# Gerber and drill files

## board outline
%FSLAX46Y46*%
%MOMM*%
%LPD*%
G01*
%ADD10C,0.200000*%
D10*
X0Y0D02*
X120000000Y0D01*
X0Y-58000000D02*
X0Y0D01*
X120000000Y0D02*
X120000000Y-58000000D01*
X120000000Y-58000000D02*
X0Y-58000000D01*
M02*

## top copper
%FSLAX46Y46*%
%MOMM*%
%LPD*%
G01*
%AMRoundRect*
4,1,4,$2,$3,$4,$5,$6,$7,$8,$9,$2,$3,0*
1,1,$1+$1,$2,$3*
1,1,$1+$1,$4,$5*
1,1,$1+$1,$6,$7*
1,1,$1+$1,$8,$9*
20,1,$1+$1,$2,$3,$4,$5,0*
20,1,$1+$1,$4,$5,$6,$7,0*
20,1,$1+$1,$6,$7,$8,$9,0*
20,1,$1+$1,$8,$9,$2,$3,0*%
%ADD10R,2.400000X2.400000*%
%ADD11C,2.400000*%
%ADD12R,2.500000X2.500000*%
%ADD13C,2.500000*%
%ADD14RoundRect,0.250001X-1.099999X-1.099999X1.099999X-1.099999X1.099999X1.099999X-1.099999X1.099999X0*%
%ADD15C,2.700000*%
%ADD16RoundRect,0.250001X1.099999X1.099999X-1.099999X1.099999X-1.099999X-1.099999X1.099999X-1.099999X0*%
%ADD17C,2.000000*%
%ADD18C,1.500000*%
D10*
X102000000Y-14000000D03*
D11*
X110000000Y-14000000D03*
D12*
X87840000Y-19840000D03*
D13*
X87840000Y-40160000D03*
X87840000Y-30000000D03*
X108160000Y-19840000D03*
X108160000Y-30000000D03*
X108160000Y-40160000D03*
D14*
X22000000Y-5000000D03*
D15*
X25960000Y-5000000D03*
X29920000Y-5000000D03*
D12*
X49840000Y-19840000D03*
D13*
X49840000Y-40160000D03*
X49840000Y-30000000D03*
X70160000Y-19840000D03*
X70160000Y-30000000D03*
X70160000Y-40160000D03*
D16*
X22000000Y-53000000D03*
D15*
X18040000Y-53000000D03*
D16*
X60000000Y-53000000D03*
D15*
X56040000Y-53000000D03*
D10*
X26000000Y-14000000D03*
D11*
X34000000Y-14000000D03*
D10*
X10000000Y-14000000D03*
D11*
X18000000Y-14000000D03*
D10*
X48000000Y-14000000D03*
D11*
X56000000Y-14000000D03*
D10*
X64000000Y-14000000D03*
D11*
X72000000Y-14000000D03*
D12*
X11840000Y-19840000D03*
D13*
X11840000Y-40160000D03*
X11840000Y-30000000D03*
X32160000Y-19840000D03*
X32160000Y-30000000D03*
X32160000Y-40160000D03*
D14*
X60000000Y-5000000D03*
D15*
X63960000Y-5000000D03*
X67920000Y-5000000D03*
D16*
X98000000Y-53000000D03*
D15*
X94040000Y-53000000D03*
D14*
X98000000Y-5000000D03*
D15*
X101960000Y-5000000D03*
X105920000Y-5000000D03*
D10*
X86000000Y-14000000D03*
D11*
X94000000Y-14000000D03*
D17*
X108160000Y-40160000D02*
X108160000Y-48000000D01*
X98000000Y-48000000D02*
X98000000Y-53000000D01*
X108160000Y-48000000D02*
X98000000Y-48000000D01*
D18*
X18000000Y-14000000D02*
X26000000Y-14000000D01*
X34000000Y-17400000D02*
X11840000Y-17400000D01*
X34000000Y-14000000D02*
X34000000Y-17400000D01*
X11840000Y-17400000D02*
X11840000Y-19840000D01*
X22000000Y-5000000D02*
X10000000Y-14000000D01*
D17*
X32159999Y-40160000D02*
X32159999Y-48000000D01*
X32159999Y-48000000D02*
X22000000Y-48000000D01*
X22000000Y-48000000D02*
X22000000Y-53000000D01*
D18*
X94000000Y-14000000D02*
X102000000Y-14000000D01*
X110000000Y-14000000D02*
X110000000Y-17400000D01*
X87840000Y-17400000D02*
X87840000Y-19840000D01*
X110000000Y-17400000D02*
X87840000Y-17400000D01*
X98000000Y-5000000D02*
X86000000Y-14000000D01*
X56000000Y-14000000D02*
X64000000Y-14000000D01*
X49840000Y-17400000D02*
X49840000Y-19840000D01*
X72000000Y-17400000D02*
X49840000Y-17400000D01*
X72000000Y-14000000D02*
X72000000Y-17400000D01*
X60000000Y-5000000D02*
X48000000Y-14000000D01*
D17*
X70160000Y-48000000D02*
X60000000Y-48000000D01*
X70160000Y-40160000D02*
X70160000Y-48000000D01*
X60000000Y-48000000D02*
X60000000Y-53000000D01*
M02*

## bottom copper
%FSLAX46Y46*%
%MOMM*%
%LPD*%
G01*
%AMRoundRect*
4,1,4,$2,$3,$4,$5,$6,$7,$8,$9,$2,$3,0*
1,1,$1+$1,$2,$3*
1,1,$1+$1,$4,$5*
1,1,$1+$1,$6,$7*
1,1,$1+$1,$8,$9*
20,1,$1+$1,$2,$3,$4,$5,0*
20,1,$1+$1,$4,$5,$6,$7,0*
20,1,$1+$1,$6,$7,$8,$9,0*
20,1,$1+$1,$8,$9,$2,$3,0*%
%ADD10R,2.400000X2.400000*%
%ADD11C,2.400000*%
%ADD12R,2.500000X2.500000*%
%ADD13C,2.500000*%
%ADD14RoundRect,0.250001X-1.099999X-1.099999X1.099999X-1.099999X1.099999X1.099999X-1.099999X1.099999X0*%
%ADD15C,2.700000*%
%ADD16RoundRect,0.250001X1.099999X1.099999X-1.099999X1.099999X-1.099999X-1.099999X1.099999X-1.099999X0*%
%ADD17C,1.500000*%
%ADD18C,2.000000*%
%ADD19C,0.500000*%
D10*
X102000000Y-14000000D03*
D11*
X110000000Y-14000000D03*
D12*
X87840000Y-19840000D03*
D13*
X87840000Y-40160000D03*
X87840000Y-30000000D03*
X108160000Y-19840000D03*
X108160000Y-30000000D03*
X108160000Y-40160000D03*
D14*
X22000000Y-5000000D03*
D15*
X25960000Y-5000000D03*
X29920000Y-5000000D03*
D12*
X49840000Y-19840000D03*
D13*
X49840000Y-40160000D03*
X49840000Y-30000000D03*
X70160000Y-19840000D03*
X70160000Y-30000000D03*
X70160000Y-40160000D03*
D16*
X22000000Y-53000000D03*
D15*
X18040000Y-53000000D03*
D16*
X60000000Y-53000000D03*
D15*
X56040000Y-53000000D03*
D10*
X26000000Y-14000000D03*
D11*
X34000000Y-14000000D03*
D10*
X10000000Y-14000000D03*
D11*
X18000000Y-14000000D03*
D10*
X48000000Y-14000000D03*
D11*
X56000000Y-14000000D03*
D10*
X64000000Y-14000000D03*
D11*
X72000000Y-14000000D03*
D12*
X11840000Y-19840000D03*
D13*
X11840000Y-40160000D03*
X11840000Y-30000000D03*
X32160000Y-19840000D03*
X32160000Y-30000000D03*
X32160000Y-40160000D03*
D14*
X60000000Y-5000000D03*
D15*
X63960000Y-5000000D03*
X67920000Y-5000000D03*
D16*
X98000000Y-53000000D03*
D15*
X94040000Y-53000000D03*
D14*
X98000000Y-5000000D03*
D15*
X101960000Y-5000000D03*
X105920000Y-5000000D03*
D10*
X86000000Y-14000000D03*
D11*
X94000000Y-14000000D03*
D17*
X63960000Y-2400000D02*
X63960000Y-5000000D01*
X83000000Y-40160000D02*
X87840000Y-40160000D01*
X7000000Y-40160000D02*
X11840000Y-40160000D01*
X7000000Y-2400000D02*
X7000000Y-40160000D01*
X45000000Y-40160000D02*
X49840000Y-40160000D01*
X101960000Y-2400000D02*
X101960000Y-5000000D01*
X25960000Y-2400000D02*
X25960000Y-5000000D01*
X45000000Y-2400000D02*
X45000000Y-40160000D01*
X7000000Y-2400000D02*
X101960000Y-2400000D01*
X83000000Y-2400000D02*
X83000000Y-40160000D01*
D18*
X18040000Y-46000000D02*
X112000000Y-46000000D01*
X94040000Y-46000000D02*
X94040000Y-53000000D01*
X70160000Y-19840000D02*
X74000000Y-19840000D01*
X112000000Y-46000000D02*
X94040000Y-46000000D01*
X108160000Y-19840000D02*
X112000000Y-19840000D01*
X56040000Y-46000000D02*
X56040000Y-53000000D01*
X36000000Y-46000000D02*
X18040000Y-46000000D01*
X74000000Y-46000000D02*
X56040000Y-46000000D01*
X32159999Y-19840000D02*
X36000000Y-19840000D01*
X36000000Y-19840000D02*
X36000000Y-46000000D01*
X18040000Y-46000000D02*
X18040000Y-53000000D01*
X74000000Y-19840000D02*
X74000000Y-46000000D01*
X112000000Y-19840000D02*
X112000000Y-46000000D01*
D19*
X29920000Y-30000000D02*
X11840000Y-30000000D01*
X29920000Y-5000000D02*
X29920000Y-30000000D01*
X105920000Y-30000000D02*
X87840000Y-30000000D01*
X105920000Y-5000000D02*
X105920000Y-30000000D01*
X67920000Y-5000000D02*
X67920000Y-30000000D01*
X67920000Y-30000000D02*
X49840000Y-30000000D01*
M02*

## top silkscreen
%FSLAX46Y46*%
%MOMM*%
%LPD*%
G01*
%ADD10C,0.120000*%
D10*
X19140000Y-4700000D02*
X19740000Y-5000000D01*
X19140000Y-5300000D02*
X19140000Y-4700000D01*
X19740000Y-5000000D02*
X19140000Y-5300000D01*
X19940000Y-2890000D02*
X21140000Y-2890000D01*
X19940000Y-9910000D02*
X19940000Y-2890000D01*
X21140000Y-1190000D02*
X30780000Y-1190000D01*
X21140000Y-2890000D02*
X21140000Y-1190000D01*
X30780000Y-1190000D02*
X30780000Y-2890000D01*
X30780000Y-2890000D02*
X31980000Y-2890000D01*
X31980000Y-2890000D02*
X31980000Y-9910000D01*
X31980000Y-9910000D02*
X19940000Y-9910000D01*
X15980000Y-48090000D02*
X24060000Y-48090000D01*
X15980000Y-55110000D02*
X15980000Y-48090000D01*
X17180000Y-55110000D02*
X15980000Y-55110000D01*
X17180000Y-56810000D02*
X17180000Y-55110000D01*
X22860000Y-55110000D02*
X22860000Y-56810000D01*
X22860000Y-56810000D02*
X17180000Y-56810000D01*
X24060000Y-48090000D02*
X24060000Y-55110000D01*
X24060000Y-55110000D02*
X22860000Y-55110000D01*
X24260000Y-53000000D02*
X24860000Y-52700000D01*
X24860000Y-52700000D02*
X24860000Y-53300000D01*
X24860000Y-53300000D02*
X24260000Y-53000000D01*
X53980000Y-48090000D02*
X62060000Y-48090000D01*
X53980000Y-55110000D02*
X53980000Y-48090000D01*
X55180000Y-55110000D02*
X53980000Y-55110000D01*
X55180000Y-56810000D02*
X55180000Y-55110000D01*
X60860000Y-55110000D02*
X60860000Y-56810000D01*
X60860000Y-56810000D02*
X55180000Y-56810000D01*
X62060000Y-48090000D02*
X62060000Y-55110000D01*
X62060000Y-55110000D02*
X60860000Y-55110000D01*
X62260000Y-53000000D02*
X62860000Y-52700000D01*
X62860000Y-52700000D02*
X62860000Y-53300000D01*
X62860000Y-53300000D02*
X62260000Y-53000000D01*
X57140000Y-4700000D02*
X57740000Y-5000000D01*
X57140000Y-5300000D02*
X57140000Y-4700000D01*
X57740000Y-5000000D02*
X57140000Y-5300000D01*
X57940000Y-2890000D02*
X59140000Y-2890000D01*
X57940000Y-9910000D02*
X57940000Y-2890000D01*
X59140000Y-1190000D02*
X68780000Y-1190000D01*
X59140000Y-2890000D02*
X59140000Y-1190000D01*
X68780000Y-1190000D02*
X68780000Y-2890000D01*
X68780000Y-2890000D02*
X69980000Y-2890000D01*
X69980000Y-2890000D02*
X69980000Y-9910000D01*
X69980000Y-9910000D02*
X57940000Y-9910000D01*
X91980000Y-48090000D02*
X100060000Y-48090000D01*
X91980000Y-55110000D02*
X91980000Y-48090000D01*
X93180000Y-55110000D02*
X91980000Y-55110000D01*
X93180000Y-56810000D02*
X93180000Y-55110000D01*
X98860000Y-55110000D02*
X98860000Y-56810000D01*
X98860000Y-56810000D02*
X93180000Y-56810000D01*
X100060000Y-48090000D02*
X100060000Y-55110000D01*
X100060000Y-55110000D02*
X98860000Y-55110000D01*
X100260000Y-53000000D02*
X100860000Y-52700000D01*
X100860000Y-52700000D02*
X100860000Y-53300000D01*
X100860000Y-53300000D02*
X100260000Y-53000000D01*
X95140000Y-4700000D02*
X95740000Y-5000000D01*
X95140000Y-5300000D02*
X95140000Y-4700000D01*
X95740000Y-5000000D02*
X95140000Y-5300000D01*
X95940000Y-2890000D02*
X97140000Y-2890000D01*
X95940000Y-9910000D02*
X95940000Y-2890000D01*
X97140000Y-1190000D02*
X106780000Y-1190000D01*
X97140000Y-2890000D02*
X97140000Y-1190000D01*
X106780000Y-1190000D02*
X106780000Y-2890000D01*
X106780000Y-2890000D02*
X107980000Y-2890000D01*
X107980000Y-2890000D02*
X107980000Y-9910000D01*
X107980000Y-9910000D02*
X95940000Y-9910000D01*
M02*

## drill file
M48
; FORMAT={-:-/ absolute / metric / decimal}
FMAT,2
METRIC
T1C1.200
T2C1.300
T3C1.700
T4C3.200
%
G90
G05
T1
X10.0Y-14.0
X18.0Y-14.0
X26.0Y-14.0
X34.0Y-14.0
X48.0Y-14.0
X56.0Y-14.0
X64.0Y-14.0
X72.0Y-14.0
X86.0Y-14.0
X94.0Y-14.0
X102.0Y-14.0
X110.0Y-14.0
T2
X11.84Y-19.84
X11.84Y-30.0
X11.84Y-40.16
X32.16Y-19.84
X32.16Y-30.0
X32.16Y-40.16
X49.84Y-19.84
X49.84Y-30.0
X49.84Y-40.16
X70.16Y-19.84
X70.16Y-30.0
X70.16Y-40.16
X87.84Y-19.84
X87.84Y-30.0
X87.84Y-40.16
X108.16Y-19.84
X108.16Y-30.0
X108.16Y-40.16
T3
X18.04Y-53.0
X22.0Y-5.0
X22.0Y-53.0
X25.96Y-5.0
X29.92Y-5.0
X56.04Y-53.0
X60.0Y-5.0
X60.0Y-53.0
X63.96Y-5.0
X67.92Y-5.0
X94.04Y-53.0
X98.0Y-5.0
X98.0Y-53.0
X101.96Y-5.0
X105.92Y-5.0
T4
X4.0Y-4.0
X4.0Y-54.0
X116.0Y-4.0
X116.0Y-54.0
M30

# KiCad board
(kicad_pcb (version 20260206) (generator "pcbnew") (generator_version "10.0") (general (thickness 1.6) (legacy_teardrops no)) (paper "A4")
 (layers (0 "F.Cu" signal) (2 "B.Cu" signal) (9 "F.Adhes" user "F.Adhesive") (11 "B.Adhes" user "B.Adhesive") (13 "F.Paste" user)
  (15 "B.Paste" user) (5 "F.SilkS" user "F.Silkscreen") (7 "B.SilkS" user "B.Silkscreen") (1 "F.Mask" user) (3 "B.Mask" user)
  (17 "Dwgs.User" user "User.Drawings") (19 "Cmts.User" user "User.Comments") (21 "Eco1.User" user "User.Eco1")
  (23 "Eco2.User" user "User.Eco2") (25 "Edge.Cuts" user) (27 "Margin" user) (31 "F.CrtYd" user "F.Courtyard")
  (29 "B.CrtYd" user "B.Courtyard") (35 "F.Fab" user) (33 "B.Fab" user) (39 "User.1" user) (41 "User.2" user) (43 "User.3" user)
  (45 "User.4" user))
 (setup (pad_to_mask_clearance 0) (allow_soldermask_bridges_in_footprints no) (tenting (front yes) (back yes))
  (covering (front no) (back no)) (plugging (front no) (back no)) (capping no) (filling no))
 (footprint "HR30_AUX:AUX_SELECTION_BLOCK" (layer "F.Cu") (at 106 14)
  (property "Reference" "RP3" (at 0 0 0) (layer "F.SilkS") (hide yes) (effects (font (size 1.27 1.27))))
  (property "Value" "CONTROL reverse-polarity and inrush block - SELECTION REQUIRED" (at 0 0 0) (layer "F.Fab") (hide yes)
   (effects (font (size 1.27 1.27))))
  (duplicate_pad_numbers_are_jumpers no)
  (pad "1" thru_hole rect (at -4 0) (size 2.4 2.4) (drill 1.2) (layers "*.Cu") (remove_unused_layers no) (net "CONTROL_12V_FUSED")
   (thermal_bridge_angle 45))
  (pad "2" thru_hole circle (at 4 0) (size 2.4 2.4) (drill 1.2) (layers "*.Cu") (remove_unused_layers no) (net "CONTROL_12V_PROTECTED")))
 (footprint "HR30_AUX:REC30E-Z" (layer "F.Cu") (at 98 30)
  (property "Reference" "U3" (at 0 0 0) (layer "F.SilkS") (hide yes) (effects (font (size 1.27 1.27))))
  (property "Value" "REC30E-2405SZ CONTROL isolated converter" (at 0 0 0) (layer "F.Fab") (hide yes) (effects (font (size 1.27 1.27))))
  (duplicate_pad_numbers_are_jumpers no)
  (pad "1" thru_hole rect (at -10.16 -10.16) (size 2.5 2.5) (drill 1.3) (layers "*.Cu") (remove_unused_layers no)
   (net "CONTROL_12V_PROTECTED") (thermal_bridge_angle 45))
  (pad "2" thru_hole circle (at -10.16 10.16) (size 2.5 2.5) (drill 1.3) (layers "*.Cu") (remove_unused_layers no) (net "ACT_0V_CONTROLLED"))
  (pad "3" thru_hole circle (at -10.16 0) (size 2.5 2.5) (drill 1.3) (layers "*.Cu") (remove_unused_layers no) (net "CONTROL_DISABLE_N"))
  (pad "4" thru_hole circle (at 10.16 -10.16) (size 2.5 2.5) (drill 1.3) (layers "*.Cu") (remove_unused_layers no) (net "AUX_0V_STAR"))
  (pad "5" thru_hole circle (at 10.16 0) (size 2.5 2.5) (drill 1.3) (layers "*.Cu") (remove_unused_layers no))
  (pad "6" thru_hole circle (at 10.16 10.16) (size 2.5 2.5) (drill 1.3) (layers "*.Cu") (remove_unused_layers no) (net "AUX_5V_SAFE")))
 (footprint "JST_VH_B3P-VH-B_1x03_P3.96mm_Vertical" (layer "F.Cu") (at 22 5)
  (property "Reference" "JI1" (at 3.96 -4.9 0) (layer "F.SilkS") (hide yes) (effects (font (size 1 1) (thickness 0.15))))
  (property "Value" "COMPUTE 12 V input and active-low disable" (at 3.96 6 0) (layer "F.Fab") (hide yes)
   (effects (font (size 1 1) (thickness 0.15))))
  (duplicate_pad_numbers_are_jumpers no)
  (fp_line (start -2.86 -0.3) (end -2.26 0) (stroke (width 0.12) (type solid)) (layer "F.SilkS"))
  (fp_line (start -2.86 0.3) (end -2.86 -0.3) (stroke (width 0.12) (type solid)) (layer "F.SilkS"))
  (fp_line (start -2.26 0) (end -2.86 0.3) (stroke (width 0.12) (type solid)) (layer "F.SilkS"))
  (fp_line (start -2.06 -2.11) (end -0.86 -2.11) (stroke (width 0.12) (type solid)) (layer "F.SilkS"))
  (fp_line (start -2.06 4.91) (end -2.06 -2.11) (stroke (width 0.12) (type solid)) (layer "F.SilkS"))
  (fp_line (start -0.86 -3.81) (end 8.78 -3.81) (stroke (width 0.12) (type solid)) (layer "F.SilkS"))
  (fp_line (start -0.86 -2.11) (end -0.86 -3.81) (stroke (width 0.12) (type solid)) (layer "F.SilkS"))
  (fp_line (start 8.78 -3.81) (end 8.78 -2.11) (stroke (width 0.12) (type solid)) (layer "F.SilkS"))
  (fp_line (start 8.78 -2.11) (end 9.98 -2.11) (stroke (width 0.12) (type solid)) (layer "F.SilkS"))
  (fp_line (start 9.98 -2.11) (end 9.98 4.91) (stroke (width 0.12) (type solid)) (layer "F.SilkS"))
  (fp_line (start 9.98 4.91) (end -2.06 4.91) (stroke (width 0.12) (type solid)) (layer "F.SilkS"))
  (pad "1" thru_hole roundrect (at 0 0) (size 2.7 2.7) (drill 1.7) (layers "*.Cu") (remove_unused_layers no) (roundrect_rratio 0.092593)
   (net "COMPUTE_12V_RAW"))
  (pad "2" thru_hole circle (at 3.96 0) (size 2.7 2.7) (drill 1.7) (layers "*.Cu") (remove_unused_layers no) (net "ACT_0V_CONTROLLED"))
  (pad "3" thru_hole circle (at 7.92 0) (size 2.7 2.7) (drill 1.7) (layers "*.Cu") (remove_unused_layers no) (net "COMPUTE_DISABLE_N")))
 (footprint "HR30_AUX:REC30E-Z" (layer "F.Cu") (at 60 30)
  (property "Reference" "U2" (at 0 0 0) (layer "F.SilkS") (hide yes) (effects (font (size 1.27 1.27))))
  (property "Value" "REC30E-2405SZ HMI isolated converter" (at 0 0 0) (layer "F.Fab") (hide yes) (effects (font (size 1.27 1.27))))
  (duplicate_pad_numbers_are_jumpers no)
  (pad "1" thru_hole rect (at -10.16 -10.16) (size 2.5 2.5) (drill 1.3) (layers "*.Cu") (remove_unused_layers no) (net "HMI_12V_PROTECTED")
   (thermal_bridge_angle 45))
  (pad "2" thru_hole circle (at -10.16 10.16) (size 2.5 2.5) (drill 1.3) (layers "*.Cu") (remove_unused_layers no) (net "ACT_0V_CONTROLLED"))
  (pad "3" thru_hole circle (at -10.16 0) (size 2.5 2.5) (drill 1.3) (layers "*.Cu") (remove_unused_layers no) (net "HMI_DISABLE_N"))
  (pad "4" thru_hole circle (at 10.16 -10.16) (size 2.5 2.5) (drill 1.3) (layers "*.Cu") (remove_unused_layers no) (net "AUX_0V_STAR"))
  (pad "5" thru_hole circle (at 10.16 0) (size 2.5 2.5) (drill 1.3) (layers "*.Cu") (remove_unused_layers no))
  (pad "6" thru_hole circle (at 10.16 10.16) (size 2.5 2.5) (drill 1.3) (layers "*.Cu") (remove_unused_layers no) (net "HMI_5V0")))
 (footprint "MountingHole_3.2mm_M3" (layer "F.Cu") (at 4 4)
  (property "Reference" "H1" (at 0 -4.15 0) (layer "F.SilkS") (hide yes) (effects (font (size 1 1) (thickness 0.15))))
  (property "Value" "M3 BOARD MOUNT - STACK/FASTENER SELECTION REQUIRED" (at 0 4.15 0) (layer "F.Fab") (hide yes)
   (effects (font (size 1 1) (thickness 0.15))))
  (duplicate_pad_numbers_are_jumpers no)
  (pad "" np_thru_hole circle (at 0 0) (size 3.2 3.2) (drill 3.2) (layers "*.Cu")))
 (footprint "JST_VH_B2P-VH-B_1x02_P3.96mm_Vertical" (layer "F.Cu") (at 22 53 180)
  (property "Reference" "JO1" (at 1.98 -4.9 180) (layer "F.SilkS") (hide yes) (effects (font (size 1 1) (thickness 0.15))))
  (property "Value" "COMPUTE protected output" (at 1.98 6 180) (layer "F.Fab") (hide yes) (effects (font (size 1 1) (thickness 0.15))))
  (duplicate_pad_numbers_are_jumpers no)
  (fp_line (start 6.02 4.91) (end -2.06 4.91) (stroke (width 0.12) (type solid)) (layer "F.SilkS"))
  (fp_line (start 6.02 -2.11) (end 6.02 4.91) (stroke (width 0.12) (type solid)) (layer "F.SilkS"))
  (fp_line (start 4.82 -2.11) (end 6.02 -2.11) (stroke (width 0.12) (type solid)) (layer "F.SilkS"))
  (fp_line (start 4.82 -3.81) (end 4.82 -2.11) (stroke (width 0.12) (type solid)) (layer "F.SilkS"))
  (fp_line (start -0.86 -2.11) (end -0.86 -3.81) (stroke (width 0.12) (type solid)) (layer "F.SilkS"))
  (fp_line (start -0.86 -3.81) (end 4.82 -3.81) (stroke (width 0.12) (type solid)) (layer "F.SilkS"))
  (fp_line (start -2.06 4.91) (end -2.06 -2.11) (stroke (width 0.12) (type solid)) (layer "F.SilkS"))
  (fp_line (start -2.06 -2.11) (end -0.86 -2.11) (stroke (width 0.12) (type solid)) (layer "F.SilkS"))
  (fp_line (start -2.26 0) (end -2.86 0.3) (stroke (width 0.12) (type solid)) (layer "F.SilkS"))
  (fp_line (start -2.86 0.3) (end -2.86 -0.3) (stroke (width 0.12) (type solid)) (layer "F.SilkS"))
  (fp_line (start -2.86 -0.3) (end -2.26 0) (stroke (width 0.12) (type solid)) (layer "F.SilkS"))
  (pad "1" thru_hole roundrect (at 0 0 180) (size 2.7 2.7) (drill 1.7) (layers "*.Cu") (remove_unused_layers no) (roundrect_rratio 0.092593)
   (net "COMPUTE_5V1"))
  (pad "2" thru_hole circle (at 3.96 0 180) (size 2.7 2.7) (drill 1.7) (layers "*.Cu") (remove_unused_layers no) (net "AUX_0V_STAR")))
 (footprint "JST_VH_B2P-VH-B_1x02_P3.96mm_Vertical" (layer "F.Cu") (at 60 53 180)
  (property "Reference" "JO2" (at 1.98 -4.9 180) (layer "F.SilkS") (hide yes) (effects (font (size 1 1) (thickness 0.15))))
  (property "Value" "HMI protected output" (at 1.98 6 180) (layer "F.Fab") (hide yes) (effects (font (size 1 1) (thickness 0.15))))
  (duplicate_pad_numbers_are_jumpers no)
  (fp_line (start 6.02 4.91) (end -2.06 4.91) (stroke (width 0.12) (type solid)) (layer "F.SilkS"))
  (fp_line (start 6.02 -2.11) (end 6.02 4.91) (stroke (width 0.12) (type solid)) (layer "F.SilkS"))
  (fp_line (start 4.82 -2.11) (end 6.02 -2.11) (stroke (width 0.12) (type solid)) (layer "F.SilkS"))
  (fp_line (start 4.82 -3.81) (end 4.82 -2.11) (stroke (width 0.12) (type solid)) (layer "F.SilkS"))
  (fp_line (start -0.86 -2.11) (end -0.86 -3.81) (stroke (width 0.12) (type solid)) (layer "F.SilkS"))
  (fp_line (start -0.86 -3.81) (end 4.82 -3.81) (stroke (width 0.12) (type solid)) (layer "F.SilkS"))
  (fp_line (start -2.06 4.91) (end -2.06 -2.11) (stroke (width 0.12) (type solid)) (layer "F.SilkS"))
  (fp_line (start -2.06 -2.11) (end -0.86 -2.11) (stroke (width 0.12) (type solid)) (layer "F.SilkS"))
  (fp_line (start -2.26 0) (end -2.86 0.3) (stroke (width 0.12) (type solid)) (layer "F.SilkS"))
  (fp_line (start -2.86 0.3) (end -2.86 -0.3) (stroke (width 0.12) (type solid)) (layer "F.SilkS"))
  (fp_line (start -2.86 -0.3) (end -2.26 0) (stroke (width 0.12) (type solid)) (layer "F.SilkS"))
  (pad "1" thru_hole roundrect (at 0 0 180) (size 2.7 2.7) (drill 1.7) (layers "*.Cu") (remove_unused_layers no) (roundrect_rratio 0.092593)
   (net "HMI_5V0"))
  (pad "2" thru_hole circle (at 3.96 0 180) (size 2.7 2.7) (drill 1.7) (layers "*.Cu") (remove_unused_layers no) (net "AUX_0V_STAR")))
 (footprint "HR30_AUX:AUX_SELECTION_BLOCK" (layer "F.Cu") (at 30 14)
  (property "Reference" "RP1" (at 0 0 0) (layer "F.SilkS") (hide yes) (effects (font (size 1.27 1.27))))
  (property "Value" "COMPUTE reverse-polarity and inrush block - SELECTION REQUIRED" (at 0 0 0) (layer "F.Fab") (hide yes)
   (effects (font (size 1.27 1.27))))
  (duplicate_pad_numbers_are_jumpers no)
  (pad "1" thru_hole rect (at -4 0) (size 2.4 2.4) (drill 1.2) (layers "*.Cu") (remove_unused_layers no) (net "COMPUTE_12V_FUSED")
   (thermal_bridge_angle 45))
  (pad "2" thru_hole circle (at 4 0) (size 2.4 2.4) (drill 1.2) (layers "*.Cu") (remove_unused_layers no) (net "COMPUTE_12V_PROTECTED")))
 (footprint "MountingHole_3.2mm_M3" (layer "F.Cu") (at 116 54)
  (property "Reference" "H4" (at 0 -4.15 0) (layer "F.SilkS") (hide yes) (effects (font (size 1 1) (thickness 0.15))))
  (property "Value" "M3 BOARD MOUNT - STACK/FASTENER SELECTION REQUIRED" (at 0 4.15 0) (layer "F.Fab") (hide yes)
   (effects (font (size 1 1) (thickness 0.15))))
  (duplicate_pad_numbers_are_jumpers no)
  (pad "" np_thru_hole circle (at 0 0) (size 3.2 3.2) (drill 3.2) (layers "*.Cu")))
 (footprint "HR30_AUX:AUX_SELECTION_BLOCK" (layer "F.Cu") (at 14 14)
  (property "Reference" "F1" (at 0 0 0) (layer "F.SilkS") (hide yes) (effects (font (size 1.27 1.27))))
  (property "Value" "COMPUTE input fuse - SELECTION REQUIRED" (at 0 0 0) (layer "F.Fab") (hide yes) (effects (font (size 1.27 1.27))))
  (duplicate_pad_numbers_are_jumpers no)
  (pad "1" thru_hole rect (at -4 0) (size 2.4 2.4) (drill 1.2) (layers "*.Cu") (remove_unused_layers no) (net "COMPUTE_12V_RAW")
   (thermal_bridge_angle 45))
  (pad "2" thru_hole circle (at 4 0) (size 2.4 2.4) (drill 1.2) (layers "*.Cu") (remove_unused_layers no) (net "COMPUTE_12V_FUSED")))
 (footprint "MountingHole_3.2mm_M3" (layer "F.Cu") (at 116 4)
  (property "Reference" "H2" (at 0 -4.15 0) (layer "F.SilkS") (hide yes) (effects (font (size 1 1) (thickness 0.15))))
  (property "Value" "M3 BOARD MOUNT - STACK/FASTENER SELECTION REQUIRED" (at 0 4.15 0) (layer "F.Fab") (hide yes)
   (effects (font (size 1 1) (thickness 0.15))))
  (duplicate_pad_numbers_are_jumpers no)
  (pad "" np_thru_hole circle (at 0 0) (size 3.2 3.2) (drill 3.2) (layers "*.Cu")))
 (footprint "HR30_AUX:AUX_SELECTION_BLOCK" (layer "F.Cu") (at 52 14)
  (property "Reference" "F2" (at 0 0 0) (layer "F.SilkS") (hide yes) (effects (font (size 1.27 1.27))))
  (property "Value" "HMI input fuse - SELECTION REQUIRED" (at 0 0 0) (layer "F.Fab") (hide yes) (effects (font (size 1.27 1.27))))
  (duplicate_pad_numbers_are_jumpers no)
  (pad "1" thru_hole rect (at -4 0) (size 2.4 2.4) (drill 1.2) (layers "*.Cu") (remove_unused_layers no) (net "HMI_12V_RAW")
   (thermal_bridge_angle 45))
  (pad "2" thru_hole circle (at 4 0) (size 2.4 2.4) (drill 1.2) (layers "*.Cu") (remove_unused_layers no) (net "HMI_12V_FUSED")))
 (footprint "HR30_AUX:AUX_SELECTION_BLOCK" (layer "F.Cu") (at 68 14)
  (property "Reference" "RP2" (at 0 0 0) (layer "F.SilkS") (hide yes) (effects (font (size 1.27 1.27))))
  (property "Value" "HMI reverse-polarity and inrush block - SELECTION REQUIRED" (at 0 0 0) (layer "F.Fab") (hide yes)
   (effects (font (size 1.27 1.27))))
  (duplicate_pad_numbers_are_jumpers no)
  (pad "1" thru_hole rect (at -4 0) (size 2.4 2.4) (drill 1.2) (layers "*.Cu") (remove_unused_layers no) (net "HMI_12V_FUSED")
   (thermal_bridge_angle 45))
  (pad "2" thru_hole circle (at 4 0) (size 2.4 2.4) (drill 1.2) (layers "*.Cu") (remove_unused_layers no) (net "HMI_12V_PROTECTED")))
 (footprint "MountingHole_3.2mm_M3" (layer "F.Cu") (at 4 54)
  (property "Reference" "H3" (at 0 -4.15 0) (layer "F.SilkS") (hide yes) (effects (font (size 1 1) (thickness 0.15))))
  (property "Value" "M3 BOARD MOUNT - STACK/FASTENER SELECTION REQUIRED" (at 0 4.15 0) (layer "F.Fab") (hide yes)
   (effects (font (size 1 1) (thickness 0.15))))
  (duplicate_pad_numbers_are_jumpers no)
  (pad "" np_thru_hole circle (at 0 0) (size 3.2 3.2) (drill 3.2) (layers "*.Cu")))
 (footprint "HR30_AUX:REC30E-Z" (layer "F.Cu") (at 22 30)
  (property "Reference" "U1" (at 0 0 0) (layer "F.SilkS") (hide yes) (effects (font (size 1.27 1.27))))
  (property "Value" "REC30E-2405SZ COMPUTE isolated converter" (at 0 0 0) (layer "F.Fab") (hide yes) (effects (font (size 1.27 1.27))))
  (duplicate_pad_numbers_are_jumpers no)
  (pad "1" thru_hole rect (at -10.16 -10.16) (size 2.5 2.5) (drill 1.3) (layers "*.Cu") (remove_unused_layers no)
   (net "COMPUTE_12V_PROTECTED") (thermal_bridge_angle 45))
  (pad "2" thru_hole circle (at -10.16 10.16) (size 2.5 2.5) (drill 1.3) (layers "*.Cu") (remove_unused_layers no) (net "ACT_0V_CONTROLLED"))
  (pad "3" thru_hole circle (at -10.16 0) (size 2.5 2.5) (drill 1.3) (layers "*.Cu") (remove_unused_layers no) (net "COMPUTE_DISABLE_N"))
  (pad "4" thru_hole circle (at 10.16 -10.16) (size 2.5 2.5) (drill 1.3) (layers "*.Cu") (remove_unused_layers no) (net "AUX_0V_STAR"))
  (pad "5" thru_hole circle (at 10.16 0) (size 2.5 2.5) (drill 1.3) (layers "*.Cu") (remove_unused_layers no))
  (pad "6" thru_hole circle (at 10.16 10.16) (size 2.5 2.5) (drill 1.3) (layers "*.Cu") (remove_unused_layers no) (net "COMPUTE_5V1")))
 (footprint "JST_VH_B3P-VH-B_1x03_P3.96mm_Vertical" (layer "F.Cu") (at 60 5)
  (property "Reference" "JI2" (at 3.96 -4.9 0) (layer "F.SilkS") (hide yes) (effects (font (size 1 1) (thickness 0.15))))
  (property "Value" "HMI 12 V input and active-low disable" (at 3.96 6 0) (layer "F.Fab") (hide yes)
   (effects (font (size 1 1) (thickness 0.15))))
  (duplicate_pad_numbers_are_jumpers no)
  (fp_line (start -2.86 -0.3) (end -2.26 0) (stroke (width 0.12) (type solid)) (layer "F.SilkS"))
  (fp_line (start -2.86 0.3) (end -2.86 -0.3) (stroke (width 0.12) (type solid)) (layer "F.SilkS"))
  (fp_line (start -2.26 0) (end -2.86 0.3) (stroke (width 0.12) (type solid)) (layer "F.SilkS"))
  (fp_line (start -2.06 -2.11) (end -0.86 -2.11) (stroke (width 0.12) (type solid)) (layer "F.SilkS"))
  (fp_line (start -2.06 4.91) (end -2.06 -2.11) (stroke (width 0.12) (type solid)) (layer "F.SilkS"))
  (fp_line (start -0.86 -3.81) (end 8.78 -3.81) (stroke (width 0.12) (type solid)) (layer "F.SilkS"))
  (fp_line (start -0.86 -2.11) (end -0.86 -3.81) (stroke (width 0.12) (type solid)) (layer "F.SilkS"))
  (fp_line (start 8.78 -3.81) (end 8.78 -2.11) (stroke (width 0.12) (type solid)) (layer "F.SilkS"))
  (fp_line (start 8.78 -2.11) (end 9.98 -2.11) (stroke (width 0.12) (type solid)) (layer "F.SilkS"))
  (fp_line (start 9.98 -2.11) (end 9.98 4.91) (stroke (width 0.12) (type solid)) (layer "F.SilkS"))
  (fp_line (start 9.98 4.91) (end -2.06 4.91) (stroke (width 0.12) (type solid)) (layer "F.SilkS"))
  (pad "1" thru_hole roundrect (at 0 0) (size 2.7 2.7) (drill 1.7) (layers "*.Cu") (remove_unused_layers no) (roundrect_rratio 0.092593)
   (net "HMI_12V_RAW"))
  (pad "2" thru_hole circle (at 3.96 0) (size 2.7 2.7) (drill 1.7) (layers "*.Cu") (remove_unused_layers no) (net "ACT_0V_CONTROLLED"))
  (pad "3" thru_hole circle (at 7.92 0) (size 2.7 2.7) (drill 1.7) (layers "*.Cu") (remove_unused_layers no) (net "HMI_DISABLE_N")))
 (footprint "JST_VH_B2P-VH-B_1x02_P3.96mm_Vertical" (layer "F.Cu") (at 98 53 180)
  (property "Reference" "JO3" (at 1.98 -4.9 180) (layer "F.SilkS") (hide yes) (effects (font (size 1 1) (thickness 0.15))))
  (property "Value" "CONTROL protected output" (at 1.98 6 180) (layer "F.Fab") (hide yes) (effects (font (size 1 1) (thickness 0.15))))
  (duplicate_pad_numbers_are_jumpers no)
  (fp_line (start 6.02 4.91) (end -2.06 4.91) (stroke (width 0.12) (type solid)) (layer "F.SilkS"))
  (fp_line (start 6.02 -2.11) (end 6.02 4.91) (stroke (width 0.12) (type solid)) (layer "F.SilkS"))
  (fp_line (start 4.82 -2.11) (end 6.02 -2.11) (stroke (width 0.12) (type solid)) (layer "F.SilkS"))
  (fp_line (start 4.82 -3.81) (end 4.82 -2.11) (stroke (width 0.12) (type solid)) (layer "F.SilkS"))
  (fp_line (start -0.86 -2.11) (end -0.86 -3.81) (stroke (width 0.12) (type solid)) (layer "F.SilkS"))
  (fp_line (start -0.86 -3.81) (end 4.82 -3.81) (stroke (width 0.12) (type solid)) (layer "F.SilkS"))
  (fp_line (start -2.06 4.91) (end -2.06 -2.11) (stroke (width 0.12) (type solid)) (layer "F.SilkS"))
  (fp_line (start -2.06 -2.11) (end -0.86 -2.11) (stroke (width 0.12) (type solid)) (layer "F.SilkS"))
  (fp_line (start -2.26 0) (end -2.86 0.3) (stroke (width 0.12) (type solid)) (layer "F.SilkS"))
  (fp_line (start -2.86 0.3) (end -2.86 -0.3) (stroke (width 0.12) (type solid)) (layer "F.SilkS"))
  (fp_line (start -2.86 -0.3) (end -2.26 0) (stroke (width 0.12) (type solid)) (layer "F.SilkS"))
  (pad "1" thru_hole roundrect (at 0 0 180) (size 2.7 2.7) (drill 1.7) (layers "*.Cu") (remove_unused_layers no) (roundrect_rratio 0.092593)
   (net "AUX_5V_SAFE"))
  (pad "2" thru_hole circle (at 3.96 0 180) (size 2.7 2.7) (drill 1.7) (layers "*.Cu") (remove_unused_layers no) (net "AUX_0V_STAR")))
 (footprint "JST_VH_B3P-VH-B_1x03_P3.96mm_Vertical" (layer "F.Cu") (at 98 5)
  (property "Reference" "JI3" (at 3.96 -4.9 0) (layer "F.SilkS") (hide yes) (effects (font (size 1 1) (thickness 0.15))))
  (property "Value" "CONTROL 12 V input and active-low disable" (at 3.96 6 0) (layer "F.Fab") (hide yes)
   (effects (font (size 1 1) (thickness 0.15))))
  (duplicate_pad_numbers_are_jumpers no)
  (fp_line (start -2.86 -0.3) (end -2.26 0) (stroke (width 0.12) (type solid)) (layer "F.SilkS"))
  (fp_line (start -2.86 0.3) (end -2.86 -0.3) (stroke (width 0.12) (type solid)) (layer "F.SilkS"))
  (fp_line (start -2.26 0) (end -2.86 0.3) (stroke (width 0.12) (type solid)) (layer "F.SilkS"))
  (fp_line (start -2.06 -2.11) (end -0.86 -2.11) (stroke (width 0.12) (type solid)) (layer "F.SilkS"))
  (fp_line (start -2.06 4.91) (end -2.06 -2.11) (stroke (width 0.12) (type solid)) (layer "F.SilkS"))
  (fp_line (start -0.86 -3.81) (end 8.78 -3.81) (stroke (width 0.12) (type solid)) (layer "F.SilkS"))
  (fp_line (start -0.86 -2.11) (end -0.86 -3.81) (stroke (width 0.12) (type solid)) (layer "F.SilkS"))
  (fp_line (start 8.78 -3.81) (end 8.78 -2.11) (stroke (width 0.12) (type solid)) (layer "F.SilkS"))
  (fp_line (start 8.78 -2.11) (end 9.98 -2.11) (stroke (width 0.12) (type solid)) (layer "F.SilkS"))
  (fp_line (start 9.98 -2.11) (end 9.98 4.91) (stroke (width 0.12) (type solid)) (layer "F.SilkS"))
  (fp_line (start 9.98 4.91) (end -2.06 4.91) (stroke (width 0.12) (type solid)) (layer "F.SilkS"))
  (pad "1" thru_hole roundrect (at 0 0) (size 2.7 2.7) (drill 1.7) (layers "*.Cu") (remove_unused_layers no) (roundrect_rratio 0.092593)
   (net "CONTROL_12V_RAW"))
  (pad "2" thru_hole circle (at 3.96 0) (size 2.7 2.7) (drill 1.7) (layers "*.Cu") (remove_unused_layers no) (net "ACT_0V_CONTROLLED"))
  (pad "3" thru_hole circle (at 7.92 0) (size 2.7 2.7) (drill 1.7) (layers "*.Cu") (remove_unused_layers no) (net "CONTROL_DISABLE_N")))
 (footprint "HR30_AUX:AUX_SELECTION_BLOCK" (layer "F.Cu") (at 90 14)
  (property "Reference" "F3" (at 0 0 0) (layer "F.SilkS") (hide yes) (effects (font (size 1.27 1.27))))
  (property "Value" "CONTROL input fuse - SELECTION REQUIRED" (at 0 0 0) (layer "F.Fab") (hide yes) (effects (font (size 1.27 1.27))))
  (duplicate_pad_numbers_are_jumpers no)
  (pad "1" thru_hole rect (at -4 0) (size 2.4 2.4) (drill 1.2) (layers "*.Cu") (remove_unused_layers no) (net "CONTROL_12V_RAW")
   (thermal_bridge_angle 45))
  (pad "2" thru_hole circle (at 4 0) (size 2.4 2.4) (drill 1.2) (layers "*.Cu") (remove_unused_layers no) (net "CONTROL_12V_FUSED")))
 (gr_line (start 0 0) (end 120 0) (stroke (width 0.2) (type default)) (layer "Edge.Cuts"))
 (gr_line (start 0 58) (end 0 0) (stroke (width 0.2) (type default)) (layer "Edge.Cuts"))
 (gr_line (start 120 0) (end 120 58) (stroke (width 0.2) (type default)) (layer "Edge.Cuts"))
 (gr_line (start 120 58) (end 0 58) (stroke (width 0.2) (type default)) (layer "Edge.Cuts"))
 (segment (start 63.96 2.4) (end 63.96 5) (width 1.5) (layer "B.Cu") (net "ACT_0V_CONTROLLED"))
 (segment (start 83 40.16) (end 87.84 40.16) (width 1.5) (layer "B.Cu") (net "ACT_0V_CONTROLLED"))
 (segment (start 7 40.16) (end 11.84 40.16) (width 1.5) (layer "B.Cu") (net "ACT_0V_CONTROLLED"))
 (segment (start 7 2.4) (end 7 40.16) (width 1.5) (layer "B.Cu") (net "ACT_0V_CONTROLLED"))
 (segment (start 45 40.16) (end 49.84 40.16) (width 1.5) (layer "B.Cu") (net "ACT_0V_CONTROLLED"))
 (segment (start 101.96 2.4) (end 101.96 5) (width 1.5) (layer "B.Cu") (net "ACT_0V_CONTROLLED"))
 (segment (start 25.96 2.4) (end 25.96 5) (width 1.5) (layer "B.Cu") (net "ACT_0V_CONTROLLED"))
 (segment (start 45 2.4) (end 45 40.16) (width 1.5) (layer "B.Cu") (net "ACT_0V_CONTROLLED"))
 (segment (start 7 2.4) (end 101.96 2.4) (width 1.5) (layer "B.Cu") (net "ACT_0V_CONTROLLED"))
 (segment (start 83 2.4) (end 83 40.16) (width 1.5) (layer "B.Cu") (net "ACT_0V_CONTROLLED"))
 (segment (start 18.04 46) (end 112 46) (width 2) (layer "B.Cu") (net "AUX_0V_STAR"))
 (segment (start 94.04 46) (end 94.04 53) (width 2) (layer "B.Cu") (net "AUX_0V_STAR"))
 (segment (start 70.16 19.84) (end 74 19.84) (width 2) (layer "B.Cu") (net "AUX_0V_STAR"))
 (segment (start 112 46) (end 94.04 46) (width 2) (layer "B.Cu") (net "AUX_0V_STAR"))
 (segment (start 108.16 19.84) (end 112 19.84) (width 2) (layer "B.Cu") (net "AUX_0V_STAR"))
 (segment (start 56.04 46) (end 56.04 53) (width 2) (layer "B.Cu") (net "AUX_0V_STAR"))
 (segment (start 36 46) (end 18.04 46) (width 2) (layer "B.Cu") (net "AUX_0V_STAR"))
 (segment (start 74 46) (end 56.04 46) (width 2) (layer "B.Cu") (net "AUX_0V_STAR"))
 (segment (start 32.159999 19.84) (end 36 19.84) (width 2) (layer "B.Cu") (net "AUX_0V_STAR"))
 (segment (start 36 19.84) (end 36 46) (width 2) (layer "B.Cu") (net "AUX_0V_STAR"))
 (segment (start 18.04 46) (end 18.04 53) (width 2) (layer "B.Cu") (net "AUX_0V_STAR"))
 (segment (start 74 19.84) (end 74 46) (width 2) (layer "B.Cu") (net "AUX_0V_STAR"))
 (segment (start 112 19.84) (end 112 46) (width 2) (layer "B.Cu") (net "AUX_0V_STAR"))
 (segment (start 108.16 40.16) (end 108.16 48) (width 2) (layer "F.Cu") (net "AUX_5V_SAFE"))
 (segment (start 98 48) (end 98 53) (width 2) (layer "F.Cu") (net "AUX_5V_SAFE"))
 (segment (start 108.16 48) (end 98 48) (width 2) (layer "F.Cu") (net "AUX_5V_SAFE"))
 (segment (start 18 14) (end 26 14) (width 1.5) (layer "F.Cu") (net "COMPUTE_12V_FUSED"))
 (segment (start 34 17.4) (end 11.84 17.4) (width 1.5) (layer "F.Cu") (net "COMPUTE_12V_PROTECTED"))
 (segment (start 34 14) (end 34 17.4) (width 1.5) (layer "F.Cu") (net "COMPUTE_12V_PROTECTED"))
 (segment (start 11.84 17.4) (end 11.84 19.84) (width 1.5) (layer "F.Cu") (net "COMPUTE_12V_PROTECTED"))
 (segment (start 22 5) (end 10 14) (width 1.5) (layer "F.Cu") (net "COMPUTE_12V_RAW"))
 (segment (start 32.159999 40.16) (end 32.159999 48) (width 2) (layer "F.Cu") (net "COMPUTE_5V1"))
 (segment (start 32.159999 48) (end 22 48) (width 2) (layer "F.Cu") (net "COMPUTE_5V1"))
 (segment (start 22 48) (end 22 53) (width 2) (layer "F.Cu") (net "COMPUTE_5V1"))
 (segment (start 29.92 30) (end 11.84 30) (width 0.5) (layer "B.Cu") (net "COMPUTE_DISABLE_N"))
 (segment (start 29.92 5) (end 29.92 30) (width 0.5) (layer "B.Cu") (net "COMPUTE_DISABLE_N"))
 (segment (start 94 14) (end 102 14) (width 1.5) (layer "F.Cu") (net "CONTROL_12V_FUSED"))
 (segment (start 110 14) (end 110 17.4) (width 1.5) (layer "F.Cu") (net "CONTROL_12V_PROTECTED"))
 (segment (start 87.84 17.4) (end 87.84 19.84) (width 1.5) (layer "F.Cu") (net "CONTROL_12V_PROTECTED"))
 (segment (start 110 17.4) (end 87.84 17.4) (width 1.5) (layer "F.Cu") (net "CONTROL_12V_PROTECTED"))
 (segment (start 98 5) (end 86 14) (width 1.5) (layer "F.Cu") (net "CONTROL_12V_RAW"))
 (segment (start 105.92 30) (end 87.84 30) (width 0.5) (layer "B.Cu") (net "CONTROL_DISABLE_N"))
 (segment (start 105.92 5) (end 105.92 30) (width 0.5) (layer "B.Cu") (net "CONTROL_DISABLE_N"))
 (segment (start 56 14) (end 64 14) (width 1.5) (layer "F.Cu") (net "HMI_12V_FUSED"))
 (segment (start 49.84 17.4) (end 49.84 19.84) (width 1.5) (layer "F.Cu") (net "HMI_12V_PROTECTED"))
 (segment (start 72 17.4) (end 49.84 17.4) (width 1.5) (layer "F.Cu") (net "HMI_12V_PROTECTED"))
 (segment (start 72 14) (end 72 17.4) (width 1.5) (layer "F.Cu") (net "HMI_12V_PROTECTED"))
 (segment (start 60 5) (end 48 14) (width 1.5) (layer "F.Cu") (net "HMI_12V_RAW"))
 (segment (start 70.16 48) (end 60 48) (width 2) (layer "F.Cu") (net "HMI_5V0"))
 (segment (start 70.16 40.16) (end 70.16 48) (width 2) (layer "F.Cu") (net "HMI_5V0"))
 (segment (start 60 48) (end 60 53) (width 2) (layer "F.Cu") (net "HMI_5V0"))
 (segment (start 67.92 5) (end 67.92 30) (width 0.5) (layer "B.Cu") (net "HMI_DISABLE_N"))
 (segment (start 67.92 30) (end 49.84 30) (width 0.5) (layer "B.Cu") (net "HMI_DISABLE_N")))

